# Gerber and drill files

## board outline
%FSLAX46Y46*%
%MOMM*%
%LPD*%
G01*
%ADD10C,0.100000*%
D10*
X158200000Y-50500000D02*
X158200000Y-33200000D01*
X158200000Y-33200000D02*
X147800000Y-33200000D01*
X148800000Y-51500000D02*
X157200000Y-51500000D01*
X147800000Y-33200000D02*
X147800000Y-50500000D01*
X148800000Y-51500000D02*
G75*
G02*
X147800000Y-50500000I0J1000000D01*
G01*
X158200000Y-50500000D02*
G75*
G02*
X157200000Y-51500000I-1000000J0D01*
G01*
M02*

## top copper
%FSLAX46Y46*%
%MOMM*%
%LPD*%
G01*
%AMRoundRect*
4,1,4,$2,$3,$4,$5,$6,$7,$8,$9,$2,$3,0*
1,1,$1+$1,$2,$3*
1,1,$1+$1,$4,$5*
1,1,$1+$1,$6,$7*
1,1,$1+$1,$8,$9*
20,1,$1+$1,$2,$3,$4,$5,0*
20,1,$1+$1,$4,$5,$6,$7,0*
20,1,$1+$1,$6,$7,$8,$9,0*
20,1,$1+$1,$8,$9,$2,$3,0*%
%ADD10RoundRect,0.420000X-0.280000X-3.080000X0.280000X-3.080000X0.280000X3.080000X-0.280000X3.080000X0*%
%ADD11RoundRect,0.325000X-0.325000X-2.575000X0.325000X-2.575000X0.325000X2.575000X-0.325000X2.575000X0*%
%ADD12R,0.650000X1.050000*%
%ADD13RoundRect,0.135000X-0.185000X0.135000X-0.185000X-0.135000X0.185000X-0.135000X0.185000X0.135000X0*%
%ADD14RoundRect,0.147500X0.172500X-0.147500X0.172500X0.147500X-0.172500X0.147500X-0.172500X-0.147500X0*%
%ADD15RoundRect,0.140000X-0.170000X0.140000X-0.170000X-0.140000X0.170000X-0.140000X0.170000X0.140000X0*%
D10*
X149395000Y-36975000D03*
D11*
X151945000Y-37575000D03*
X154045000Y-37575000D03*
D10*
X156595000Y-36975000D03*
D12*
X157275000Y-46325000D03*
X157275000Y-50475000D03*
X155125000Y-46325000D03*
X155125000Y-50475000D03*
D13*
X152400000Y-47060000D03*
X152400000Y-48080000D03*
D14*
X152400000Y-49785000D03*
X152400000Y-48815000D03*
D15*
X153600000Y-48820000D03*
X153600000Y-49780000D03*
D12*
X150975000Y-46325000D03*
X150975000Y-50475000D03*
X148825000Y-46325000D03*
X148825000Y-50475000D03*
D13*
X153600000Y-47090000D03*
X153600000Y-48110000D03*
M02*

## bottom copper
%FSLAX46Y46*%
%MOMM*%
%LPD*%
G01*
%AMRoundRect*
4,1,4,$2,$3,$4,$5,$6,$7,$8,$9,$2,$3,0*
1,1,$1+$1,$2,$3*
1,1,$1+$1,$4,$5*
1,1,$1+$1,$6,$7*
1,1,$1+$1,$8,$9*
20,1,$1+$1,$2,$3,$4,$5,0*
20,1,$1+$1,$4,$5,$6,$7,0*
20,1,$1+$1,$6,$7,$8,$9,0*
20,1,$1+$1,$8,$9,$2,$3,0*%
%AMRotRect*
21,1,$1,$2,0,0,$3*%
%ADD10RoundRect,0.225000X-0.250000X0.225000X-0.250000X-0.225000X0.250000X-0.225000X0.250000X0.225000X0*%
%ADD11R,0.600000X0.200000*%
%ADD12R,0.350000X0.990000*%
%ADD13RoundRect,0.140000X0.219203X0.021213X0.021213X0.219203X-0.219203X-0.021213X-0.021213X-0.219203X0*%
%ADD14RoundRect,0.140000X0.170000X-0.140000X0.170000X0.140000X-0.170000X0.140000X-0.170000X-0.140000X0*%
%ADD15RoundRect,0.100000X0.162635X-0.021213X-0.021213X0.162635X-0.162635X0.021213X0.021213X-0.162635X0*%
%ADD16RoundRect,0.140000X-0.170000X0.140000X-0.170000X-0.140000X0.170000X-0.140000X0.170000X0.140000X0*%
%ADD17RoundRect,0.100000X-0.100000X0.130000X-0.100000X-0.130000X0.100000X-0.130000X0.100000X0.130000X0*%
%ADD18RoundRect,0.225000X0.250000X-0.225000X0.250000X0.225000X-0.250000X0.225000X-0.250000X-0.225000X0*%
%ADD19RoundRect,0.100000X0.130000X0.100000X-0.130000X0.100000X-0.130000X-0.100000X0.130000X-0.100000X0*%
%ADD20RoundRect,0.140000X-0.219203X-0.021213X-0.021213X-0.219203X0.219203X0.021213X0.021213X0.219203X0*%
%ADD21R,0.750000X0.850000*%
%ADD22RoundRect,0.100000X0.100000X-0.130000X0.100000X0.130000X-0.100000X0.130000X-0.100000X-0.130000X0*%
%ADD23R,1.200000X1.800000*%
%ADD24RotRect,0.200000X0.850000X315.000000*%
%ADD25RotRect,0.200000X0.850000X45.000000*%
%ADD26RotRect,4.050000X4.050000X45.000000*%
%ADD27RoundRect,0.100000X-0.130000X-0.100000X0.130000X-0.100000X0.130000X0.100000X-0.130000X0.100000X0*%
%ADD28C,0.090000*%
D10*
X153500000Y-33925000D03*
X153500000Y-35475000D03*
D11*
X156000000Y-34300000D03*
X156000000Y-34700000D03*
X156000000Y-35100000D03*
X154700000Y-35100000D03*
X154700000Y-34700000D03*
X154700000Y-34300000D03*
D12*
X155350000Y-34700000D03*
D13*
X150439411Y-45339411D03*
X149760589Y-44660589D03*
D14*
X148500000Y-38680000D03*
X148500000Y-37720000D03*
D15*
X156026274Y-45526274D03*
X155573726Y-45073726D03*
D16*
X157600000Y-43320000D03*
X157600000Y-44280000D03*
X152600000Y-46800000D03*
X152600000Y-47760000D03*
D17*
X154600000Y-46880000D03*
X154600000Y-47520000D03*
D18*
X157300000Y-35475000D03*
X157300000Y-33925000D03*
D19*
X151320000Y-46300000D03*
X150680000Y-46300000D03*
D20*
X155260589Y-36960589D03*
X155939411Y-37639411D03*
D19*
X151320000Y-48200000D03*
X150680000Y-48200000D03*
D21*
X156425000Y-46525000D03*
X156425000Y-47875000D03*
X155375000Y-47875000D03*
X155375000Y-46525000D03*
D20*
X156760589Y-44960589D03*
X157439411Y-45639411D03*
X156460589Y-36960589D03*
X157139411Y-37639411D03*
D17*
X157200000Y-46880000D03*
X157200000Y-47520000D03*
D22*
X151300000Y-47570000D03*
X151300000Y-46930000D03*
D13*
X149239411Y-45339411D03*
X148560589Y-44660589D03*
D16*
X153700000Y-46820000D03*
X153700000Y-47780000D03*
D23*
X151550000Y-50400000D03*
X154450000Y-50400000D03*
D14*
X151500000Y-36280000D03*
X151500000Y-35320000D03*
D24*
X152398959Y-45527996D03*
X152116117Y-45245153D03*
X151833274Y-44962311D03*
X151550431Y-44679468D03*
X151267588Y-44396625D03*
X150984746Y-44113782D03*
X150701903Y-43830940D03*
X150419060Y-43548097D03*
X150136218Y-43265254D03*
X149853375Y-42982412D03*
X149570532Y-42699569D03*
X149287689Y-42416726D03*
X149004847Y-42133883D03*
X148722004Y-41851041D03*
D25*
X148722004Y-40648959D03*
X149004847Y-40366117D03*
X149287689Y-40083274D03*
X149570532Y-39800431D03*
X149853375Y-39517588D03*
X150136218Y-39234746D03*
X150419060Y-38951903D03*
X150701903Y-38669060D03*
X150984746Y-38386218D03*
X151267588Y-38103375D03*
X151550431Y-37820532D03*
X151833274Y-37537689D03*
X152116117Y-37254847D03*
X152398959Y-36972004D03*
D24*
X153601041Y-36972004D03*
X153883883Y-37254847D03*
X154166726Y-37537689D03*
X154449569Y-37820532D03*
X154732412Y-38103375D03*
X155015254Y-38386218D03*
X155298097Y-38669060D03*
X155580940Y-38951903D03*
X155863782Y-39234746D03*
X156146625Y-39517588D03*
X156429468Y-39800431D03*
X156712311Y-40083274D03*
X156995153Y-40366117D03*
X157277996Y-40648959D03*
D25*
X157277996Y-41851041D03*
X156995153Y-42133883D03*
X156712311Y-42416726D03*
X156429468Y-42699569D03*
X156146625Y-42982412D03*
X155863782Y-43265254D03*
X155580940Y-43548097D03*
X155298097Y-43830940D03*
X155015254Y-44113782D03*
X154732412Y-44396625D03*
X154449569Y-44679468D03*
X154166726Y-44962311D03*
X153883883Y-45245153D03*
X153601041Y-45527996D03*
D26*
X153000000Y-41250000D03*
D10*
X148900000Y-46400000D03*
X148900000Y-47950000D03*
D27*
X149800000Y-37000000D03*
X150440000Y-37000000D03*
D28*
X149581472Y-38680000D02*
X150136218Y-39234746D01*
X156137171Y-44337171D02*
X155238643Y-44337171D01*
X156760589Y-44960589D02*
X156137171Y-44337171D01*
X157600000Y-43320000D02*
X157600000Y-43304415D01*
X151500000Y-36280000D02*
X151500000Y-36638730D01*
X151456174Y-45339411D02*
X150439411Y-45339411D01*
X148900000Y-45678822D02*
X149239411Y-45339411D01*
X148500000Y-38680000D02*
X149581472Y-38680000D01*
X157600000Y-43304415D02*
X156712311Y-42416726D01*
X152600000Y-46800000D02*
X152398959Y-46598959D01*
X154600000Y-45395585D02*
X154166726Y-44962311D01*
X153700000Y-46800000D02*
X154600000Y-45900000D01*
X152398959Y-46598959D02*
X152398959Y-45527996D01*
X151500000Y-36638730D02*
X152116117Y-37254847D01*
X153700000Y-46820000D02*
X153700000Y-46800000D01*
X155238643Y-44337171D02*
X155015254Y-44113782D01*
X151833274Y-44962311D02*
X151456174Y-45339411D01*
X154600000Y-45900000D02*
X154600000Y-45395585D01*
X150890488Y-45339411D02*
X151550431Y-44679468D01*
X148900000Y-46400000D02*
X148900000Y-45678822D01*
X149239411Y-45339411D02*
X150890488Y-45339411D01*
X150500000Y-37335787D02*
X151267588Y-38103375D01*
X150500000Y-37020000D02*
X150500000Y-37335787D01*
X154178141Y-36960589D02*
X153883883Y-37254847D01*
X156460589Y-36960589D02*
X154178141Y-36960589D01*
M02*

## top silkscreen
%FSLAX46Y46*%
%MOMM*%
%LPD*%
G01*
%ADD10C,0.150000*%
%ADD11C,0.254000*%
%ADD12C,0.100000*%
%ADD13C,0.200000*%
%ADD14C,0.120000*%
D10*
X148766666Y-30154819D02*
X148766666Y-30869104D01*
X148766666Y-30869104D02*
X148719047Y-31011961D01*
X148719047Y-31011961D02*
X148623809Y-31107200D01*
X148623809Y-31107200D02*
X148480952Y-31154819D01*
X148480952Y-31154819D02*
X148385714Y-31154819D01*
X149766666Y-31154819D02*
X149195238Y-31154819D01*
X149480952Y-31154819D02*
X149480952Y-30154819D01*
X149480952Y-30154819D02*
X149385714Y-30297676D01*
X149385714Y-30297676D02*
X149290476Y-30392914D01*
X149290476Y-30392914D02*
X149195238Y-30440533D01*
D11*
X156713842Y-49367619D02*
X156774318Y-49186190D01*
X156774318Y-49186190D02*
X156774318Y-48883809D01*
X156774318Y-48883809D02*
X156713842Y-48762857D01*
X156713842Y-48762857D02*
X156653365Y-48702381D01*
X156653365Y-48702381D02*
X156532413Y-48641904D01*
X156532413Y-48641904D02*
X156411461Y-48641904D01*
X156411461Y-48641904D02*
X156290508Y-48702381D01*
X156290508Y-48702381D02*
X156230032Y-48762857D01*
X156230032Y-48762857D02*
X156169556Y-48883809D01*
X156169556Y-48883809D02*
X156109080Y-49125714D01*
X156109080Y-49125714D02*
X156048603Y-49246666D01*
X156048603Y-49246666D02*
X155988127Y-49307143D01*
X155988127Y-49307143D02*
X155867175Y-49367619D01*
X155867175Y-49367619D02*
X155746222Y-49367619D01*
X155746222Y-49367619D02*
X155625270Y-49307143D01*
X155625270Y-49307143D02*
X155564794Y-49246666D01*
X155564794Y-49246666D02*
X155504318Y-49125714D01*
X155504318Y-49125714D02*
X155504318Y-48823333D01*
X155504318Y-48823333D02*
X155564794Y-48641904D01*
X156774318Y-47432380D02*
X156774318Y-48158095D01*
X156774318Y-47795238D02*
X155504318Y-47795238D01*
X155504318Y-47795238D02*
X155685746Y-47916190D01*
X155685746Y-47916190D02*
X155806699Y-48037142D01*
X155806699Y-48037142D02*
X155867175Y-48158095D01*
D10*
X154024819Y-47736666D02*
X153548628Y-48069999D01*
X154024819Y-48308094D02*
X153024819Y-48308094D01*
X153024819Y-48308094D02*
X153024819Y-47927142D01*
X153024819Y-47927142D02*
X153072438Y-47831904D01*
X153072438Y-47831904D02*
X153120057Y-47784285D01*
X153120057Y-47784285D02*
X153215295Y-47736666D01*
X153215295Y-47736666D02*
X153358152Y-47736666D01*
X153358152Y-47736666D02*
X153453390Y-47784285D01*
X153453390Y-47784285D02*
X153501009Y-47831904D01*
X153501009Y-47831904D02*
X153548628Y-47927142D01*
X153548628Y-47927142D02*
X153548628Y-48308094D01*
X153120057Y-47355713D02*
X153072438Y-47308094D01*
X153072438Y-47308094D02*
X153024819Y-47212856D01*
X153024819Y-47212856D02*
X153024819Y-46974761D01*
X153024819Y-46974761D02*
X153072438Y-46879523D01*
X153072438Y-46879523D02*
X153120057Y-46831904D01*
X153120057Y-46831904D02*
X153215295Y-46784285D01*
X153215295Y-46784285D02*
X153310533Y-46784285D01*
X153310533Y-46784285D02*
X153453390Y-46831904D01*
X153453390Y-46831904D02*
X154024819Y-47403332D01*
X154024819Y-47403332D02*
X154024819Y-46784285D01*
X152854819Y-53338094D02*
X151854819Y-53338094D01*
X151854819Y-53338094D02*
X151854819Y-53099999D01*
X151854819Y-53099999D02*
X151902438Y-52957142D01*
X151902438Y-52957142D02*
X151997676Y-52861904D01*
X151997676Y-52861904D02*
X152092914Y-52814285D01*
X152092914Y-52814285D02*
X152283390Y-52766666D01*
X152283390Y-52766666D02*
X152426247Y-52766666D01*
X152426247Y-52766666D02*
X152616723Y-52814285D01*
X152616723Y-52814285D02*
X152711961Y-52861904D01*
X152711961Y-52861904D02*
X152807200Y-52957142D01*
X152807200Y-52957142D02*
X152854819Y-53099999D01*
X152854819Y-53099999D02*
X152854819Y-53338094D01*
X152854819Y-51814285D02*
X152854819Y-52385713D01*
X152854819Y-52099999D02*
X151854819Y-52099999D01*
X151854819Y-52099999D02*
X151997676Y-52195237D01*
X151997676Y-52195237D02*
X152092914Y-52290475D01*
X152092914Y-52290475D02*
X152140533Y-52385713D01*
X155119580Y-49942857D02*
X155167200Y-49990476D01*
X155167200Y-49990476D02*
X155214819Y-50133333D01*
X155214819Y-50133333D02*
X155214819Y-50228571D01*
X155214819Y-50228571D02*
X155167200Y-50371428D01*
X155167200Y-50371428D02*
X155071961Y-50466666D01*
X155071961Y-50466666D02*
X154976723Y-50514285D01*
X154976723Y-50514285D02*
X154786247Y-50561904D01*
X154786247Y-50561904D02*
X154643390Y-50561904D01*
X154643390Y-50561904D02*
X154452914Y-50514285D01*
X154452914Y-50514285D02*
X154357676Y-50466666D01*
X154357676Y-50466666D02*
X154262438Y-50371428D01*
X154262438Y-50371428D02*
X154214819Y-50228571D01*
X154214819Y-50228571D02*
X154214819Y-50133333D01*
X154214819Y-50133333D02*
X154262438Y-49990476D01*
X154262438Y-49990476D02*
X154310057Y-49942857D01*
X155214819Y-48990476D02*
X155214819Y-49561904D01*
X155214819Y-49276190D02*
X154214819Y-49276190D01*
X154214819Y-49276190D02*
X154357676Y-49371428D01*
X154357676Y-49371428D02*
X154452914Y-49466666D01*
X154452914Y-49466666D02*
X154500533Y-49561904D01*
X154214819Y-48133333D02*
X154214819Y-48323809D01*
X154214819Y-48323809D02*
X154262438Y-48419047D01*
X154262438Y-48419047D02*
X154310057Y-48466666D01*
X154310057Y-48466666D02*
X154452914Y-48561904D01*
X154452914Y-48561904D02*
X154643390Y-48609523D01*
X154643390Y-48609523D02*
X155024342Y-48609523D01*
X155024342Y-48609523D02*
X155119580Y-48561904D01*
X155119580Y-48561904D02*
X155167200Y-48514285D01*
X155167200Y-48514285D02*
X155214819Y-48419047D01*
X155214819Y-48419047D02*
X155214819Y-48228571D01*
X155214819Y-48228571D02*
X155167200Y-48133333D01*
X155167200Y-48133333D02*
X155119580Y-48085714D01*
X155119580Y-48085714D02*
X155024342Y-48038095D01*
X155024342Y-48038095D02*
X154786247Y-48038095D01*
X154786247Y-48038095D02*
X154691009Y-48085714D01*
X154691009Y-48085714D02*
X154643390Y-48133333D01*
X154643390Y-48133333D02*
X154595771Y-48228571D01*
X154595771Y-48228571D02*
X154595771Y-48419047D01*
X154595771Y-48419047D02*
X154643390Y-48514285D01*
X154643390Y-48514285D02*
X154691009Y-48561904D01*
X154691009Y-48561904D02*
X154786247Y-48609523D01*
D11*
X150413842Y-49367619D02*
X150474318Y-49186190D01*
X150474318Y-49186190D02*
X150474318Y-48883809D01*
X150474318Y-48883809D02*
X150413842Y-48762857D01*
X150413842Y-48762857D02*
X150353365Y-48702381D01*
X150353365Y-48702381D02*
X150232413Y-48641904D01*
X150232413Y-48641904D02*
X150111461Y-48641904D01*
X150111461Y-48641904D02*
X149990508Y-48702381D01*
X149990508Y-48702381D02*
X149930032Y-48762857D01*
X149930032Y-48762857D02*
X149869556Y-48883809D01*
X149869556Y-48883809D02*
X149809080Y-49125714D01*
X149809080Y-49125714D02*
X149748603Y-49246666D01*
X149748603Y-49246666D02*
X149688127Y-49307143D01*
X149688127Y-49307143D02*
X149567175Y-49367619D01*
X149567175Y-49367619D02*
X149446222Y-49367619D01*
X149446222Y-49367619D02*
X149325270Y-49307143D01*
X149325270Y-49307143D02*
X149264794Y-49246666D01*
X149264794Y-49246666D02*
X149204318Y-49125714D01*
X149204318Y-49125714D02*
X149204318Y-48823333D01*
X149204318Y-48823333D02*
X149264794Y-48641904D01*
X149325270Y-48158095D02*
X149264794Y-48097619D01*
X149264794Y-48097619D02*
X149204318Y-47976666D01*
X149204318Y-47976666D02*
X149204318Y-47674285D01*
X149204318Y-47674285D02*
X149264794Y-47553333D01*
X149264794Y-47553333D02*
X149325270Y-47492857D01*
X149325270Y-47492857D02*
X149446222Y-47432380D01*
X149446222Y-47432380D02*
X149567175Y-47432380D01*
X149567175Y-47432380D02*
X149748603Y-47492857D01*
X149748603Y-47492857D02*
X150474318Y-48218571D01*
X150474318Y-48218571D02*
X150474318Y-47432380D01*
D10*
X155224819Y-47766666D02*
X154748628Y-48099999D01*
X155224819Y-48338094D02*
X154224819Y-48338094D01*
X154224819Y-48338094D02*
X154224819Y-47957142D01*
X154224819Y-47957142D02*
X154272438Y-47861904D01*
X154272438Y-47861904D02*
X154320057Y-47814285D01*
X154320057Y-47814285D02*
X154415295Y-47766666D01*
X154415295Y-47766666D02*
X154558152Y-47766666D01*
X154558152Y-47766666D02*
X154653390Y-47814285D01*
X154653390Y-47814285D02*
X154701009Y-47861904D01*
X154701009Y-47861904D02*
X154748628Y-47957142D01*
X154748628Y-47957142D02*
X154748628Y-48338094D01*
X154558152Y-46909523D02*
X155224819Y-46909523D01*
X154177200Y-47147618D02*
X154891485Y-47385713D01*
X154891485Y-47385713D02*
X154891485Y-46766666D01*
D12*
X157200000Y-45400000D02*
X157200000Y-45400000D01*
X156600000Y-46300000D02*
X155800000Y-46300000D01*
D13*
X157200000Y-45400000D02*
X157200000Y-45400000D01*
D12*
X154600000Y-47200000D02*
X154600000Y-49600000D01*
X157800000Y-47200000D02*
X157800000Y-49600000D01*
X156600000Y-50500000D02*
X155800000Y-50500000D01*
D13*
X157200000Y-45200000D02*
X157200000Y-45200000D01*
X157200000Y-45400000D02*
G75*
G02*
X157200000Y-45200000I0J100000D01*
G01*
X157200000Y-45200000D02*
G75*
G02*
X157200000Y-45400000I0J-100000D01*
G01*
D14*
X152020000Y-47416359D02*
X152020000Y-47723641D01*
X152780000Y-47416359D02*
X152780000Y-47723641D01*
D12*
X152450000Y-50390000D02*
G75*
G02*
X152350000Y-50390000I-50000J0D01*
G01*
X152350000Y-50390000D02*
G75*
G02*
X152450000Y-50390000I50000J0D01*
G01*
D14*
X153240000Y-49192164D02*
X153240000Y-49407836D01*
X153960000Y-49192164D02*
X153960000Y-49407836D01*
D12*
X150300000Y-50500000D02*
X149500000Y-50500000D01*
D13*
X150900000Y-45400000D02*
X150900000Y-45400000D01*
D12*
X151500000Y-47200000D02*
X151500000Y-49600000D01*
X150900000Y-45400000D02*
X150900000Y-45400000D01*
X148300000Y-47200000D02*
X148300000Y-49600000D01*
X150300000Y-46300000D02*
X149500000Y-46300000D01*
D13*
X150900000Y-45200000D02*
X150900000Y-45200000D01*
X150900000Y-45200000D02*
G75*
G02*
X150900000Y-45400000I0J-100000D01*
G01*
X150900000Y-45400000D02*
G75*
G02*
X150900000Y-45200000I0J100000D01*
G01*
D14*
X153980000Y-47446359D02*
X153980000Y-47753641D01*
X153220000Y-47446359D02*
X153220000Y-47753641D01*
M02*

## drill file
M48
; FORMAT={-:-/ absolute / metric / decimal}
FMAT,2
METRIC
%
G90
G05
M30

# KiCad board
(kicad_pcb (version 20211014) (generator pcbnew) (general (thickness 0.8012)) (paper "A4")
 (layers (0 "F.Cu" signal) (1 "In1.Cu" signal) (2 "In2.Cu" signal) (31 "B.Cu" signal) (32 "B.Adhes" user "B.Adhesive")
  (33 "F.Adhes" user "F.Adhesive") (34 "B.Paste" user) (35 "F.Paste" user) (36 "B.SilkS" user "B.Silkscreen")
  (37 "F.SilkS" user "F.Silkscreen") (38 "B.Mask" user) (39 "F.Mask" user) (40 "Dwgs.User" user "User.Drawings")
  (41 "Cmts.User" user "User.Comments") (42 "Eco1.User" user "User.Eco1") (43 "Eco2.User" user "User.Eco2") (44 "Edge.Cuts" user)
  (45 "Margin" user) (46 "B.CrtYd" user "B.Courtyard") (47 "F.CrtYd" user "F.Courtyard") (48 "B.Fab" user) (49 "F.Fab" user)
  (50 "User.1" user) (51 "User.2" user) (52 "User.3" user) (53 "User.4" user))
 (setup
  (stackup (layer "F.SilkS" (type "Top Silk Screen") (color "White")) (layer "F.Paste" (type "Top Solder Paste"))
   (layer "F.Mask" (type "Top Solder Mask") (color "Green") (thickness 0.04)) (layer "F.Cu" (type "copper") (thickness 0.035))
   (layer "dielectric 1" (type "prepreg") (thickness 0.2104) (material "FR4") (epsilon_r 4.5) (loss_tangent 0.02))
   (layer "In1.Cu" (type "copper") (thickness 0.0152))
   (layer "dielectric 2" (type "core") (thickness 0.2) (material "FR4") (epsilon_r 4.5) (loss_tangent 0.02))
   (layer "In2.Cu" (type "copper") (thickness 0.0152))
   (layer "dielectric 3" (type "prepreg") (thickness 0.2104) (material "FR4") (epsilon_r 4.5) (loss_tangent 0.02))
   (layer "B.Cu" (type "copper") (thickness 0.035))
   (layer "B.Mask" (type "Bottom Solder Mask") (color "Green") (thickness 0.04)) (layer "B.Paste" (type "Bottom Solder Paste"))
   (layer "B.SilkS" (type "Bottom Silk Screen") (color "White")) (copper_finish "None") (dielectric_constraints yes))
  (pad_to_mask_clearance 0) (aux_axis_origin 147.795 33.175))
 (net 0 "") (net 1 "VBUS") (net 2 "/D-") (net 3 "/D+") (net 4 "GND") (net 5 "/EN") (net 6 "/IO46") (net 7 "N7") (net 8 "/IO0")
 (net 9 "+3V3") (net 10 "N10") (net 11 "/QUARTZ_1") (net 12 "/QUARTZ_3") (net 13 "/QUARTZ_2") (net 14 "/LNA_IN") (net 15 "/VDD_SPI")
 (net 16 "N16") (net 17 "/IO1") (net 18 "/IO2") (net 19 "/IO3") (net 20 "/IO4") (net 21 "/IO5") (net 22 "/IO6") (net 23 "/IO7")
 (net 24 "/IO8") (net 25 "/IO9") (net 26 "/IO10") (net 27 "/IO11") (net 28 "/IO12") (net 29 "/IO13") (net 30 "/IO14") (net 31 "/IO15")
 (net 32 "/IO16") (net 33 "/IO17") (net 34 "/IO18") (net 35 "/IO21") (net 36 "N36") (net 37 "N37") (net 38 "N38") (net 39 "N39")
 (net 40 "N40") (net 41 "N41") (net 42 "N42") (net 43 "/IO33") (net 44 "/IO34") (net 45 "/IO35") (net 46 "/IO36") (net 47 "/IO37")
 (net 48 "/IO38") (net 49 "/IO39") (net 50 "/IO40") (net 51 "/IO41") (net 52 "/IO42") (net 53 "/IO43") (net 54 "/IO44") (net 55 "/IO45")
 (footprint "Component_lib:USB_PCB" (layer "F.Cu") (at 152.995 44.375)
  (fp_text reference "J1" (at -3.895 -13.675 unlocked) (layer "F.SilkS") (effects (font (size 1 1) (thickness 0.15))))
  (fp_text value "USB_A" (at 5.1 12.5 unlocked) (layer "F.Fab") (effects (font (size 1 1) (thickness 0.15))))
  (pad "1" smd roundrect (at -3.6 -7.4) (size 1.4 7) (layers "F.Cu" "F.Paste" "F.Mask") (roundrect_rratio 0.3) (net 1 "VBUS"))
  (pad "2" smd roundrect (at -1.05 -6.8) (size 1.3 5.8) (layers "F.Cu" "F.Paste" "F.Mask") (roundrect_rratio 0.25) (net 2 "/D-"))
  (pad "3" smd roundrect (at 1.05 -6.8) (size 1.3 5.8) (layers "F.Cu" "F.Paste" "F.Mask") (roundrect_rratio 0.25) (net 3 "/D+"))
  (pad "4" smd roundrect (at 3.6 -7.4) (size 1.4 7) (layers "F.Cu" "F.Paste" "F.Mask") (roundrect_rratio 0.3) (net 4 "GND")))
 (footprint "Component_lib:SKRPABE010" (layer "F.Cu") (at 156.2 48.4 -90)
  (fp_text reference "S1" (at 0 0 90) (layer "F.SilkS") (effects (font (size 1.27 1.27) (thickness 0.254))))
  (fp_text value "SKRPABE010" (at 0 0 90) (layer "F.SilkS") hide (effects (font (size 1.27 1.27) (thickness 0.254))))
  (fp_line (start -3 -1) (end -3 -1) (layer "F.SilkS") (width 0.1))
  (fp_line (start -2.1 -0.4) (end -2.1 0.4) (layer "F.SilkS") (width 0.1))
  (fp_line (start -3 -1) (end -3 -1) (layer "F.SilkS") (width 0.2))
  (fp_line (start -1.2 1.6) (end 1.2 1.6) (layer "F.SilkS") (width 0.1))
  (fp_line (start -1.2 -1.6) (end 1.2 -1.6) (layer "F.SilkS") (width 0.1))
  (fp_line (start 2.1 -0.4) (end 2.1 0.4) (layer "F.SilkS") (width 0.1))
  (fp_line (start -3.2 -1) (end -3.2 -1) (layer "F.SilkS") (width 0.2))
  (fp_arc (start -3 -1) (mid -3.1 -0.9) (end -3.2 -1) (layer "F.SilkS") (width 0.2))
  (fp_arc (start -3.2 -1) (mid -3.1 -1.1) (end -3 -1) (layer "F.SilkS") (width 0.2))
  (pad "1" smd rect (at -2.075 -1.075) (size 0.65 1.05) (layers "F.Cu" "F.Paste" "F.Mask") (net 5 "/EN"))
  (pad "2" smd rect (at 2.075 -1.075) (size 0.65 1.05) (layers "F.Cu" "F.Paste" "F.Mask") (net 4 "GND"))
  (pad "3" smd rect (at -2.075 1.075) (size 0.65 1.05) (layers "F.Cu" "F.Paste" "F.Mask"))
  (pad "4" smd rect (at 2.075 1.075) (size 0.65 1.05) (layers "F.Cu" "F.Paste" "F.Mask")))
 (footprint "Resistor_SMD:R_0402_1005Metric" (layer "F.Cu") (at 152.4 47.57 -90)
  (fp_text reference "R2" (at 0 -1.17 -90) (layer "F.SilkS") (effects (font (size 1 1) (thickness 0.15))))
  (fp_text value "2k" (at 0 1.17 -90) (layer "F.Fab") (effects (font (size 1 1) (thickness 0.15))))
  (fp_line (start -0.153641 0.38) (end 0.153641 0.38) (layer "F.SilkS") (width 0.12))
  (fp_line (start -0.153641 -0.38) (end 0.153641 -0.38) (layer "F.SilkS") (width 0.12))
  (pad "1" smd roundrect (at -0.51 0 270) (size 0.54 0.64) (layers "F.Cu" "F.Paste" "F.Mask") (roundrect_rratio 0.25) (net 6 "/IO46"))
  (pad "2" smd roundrect (at 0.51 0 270) (size 0.54 0.64) (layers "F.Cu" "F.Paste" "F.Mask") (roundrect_rratio 0.25) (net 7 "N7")))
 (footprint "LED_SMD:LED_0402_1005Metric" (layer "F.Cu") (at 152.4 49.3 90)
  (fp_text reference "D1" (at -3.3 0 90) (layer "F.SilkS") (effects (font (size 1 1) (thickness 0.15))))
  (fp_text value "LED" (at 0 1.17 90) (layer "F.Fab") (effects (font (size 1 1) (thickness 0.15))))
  (fp_circle (center -1.09 0) (end -1.04 0) (layer "F.SilkS") (width 0.1) (fill none))
  (pad "1" smd roundrect (at -0.485 0 90) (size 0.59 0.64) (layers "F.Cu" "F.Paste" "F.Mask") (roundrect_rratio 0.25) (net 4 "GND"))
  (pad "2" smd roundrect (at 0.485 0 90) (size 0.59 0.64) (layers "F.Cu" "F.Paste" "F.Mask") (roundrect_rratio 0.25) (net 7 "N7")))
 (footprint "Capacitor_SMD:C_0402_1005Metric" (layer "F.Cu") (at 153.6 49.3 -90)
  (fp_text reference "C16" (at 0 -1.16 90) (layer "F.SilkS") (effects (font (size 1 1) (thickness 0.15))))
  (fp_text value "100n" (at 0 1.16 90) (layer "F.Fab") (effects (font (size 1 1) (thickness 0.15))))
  (fp_line (start -0.107836 0.36) (end 0.107836 0.36) (layer "F.SilkS") (width 0.12))
  (fp_line (start -0.107836 -0.36) (end 0.107836 -0.36) (layer "F.SilkS") (width 0.12))
  (pad "1" smd roundrect (at -0.48 0 270) (size 0.56 0.62) (layers "F.Cu" "F.Paste" "F.Mask") (roundrect_rratio 0.25) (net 5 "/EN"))
  (pad "2" smd roundrect (at 0.48 0 270) (size 0.56 0.62) (layers "F.Cu" "F.Paste" "F.Mask") (roundrect_rratio 0.25) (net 4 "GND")))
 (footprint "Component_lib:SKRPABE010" (layer "F.Cu") (at 149.9 48.4 -90)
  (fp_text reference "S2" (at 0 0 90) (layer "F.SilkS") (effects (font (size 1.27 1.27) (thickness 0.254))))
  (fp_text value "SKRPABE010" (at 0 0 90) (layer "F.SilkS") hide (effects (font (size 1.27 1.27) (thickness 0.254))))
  (fp_line (start 2.1 -0.4) (end 2.1 0.4) (layer "F.SilkS") (width 0.1))
  (fp_line (start -3 -1) (end -3 -1) (layer "F.SilkS") (width 0.2))
  (fp_line (start -1.2 -1.6) (end 1.2 -1.6) (layer "F.SilkS") (width 0.1))
  (fp_line (start -3 -1) (end -3 -1) (layer "F.SilkS") (width 0.1))
  (fp_line (start -1.2 1.6) (end 1.2 1.6) (layer "F.SilkS") (width 0.1))
  (fp_line (start -2.1 -0.4) (end -2.1 0.4) (layer "F.SilkS") (width 0.1))
  (fp_line (start -3.2 -1) (end -3.2 -1) (layer "F.SilkS") (width 0.2))
  (fp_arc (start -3.2 -1) (mid -3.1 -1.1) (end -3 -1) (layer "F.SilkS") (width 0.2))
  (fp_arc (start -3 -1) (mid -3.1 -0.9) (end -3.2 -1) (layer "F.SilkS") (width 0.2))
  (pad "1" smd rect (at -2.075 -1.075) (size 0.65 1.05) (layers "F.Cu" "F.Paste" "F.Mask") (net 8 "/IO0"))
  (pad "2" smd rect (at 2.075 -1.075) (size 0.65 1.05) (layers "F.Cu" "F.Paste" "F.Mask") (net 4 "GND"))
  (pad "3" smd rect (at -2.075 1.075) (size 0.65 1.05) (layers "F.Cu" "F.Paste" "F.Mask"))
  (pad "4" smd rect (at 2.075 1.075) (size 0.65 1.05) (layers "F.Cu" "F.Paste" "F.Mask")))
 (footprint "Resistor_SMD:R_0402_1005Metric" (layer "F.Cu") (at 153.6 47.6 -90)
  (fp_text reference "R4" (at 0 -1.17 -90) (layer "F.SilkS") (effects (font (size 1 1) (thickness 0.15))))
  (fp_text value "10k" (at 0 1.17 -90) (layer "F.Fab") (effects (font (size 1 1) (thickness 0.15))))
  (fp_line (start -0.153641 -0.38) (end 0.153641 -0.38) (layer "F.SilkS") (width 0.12))
  (fp_line (start -0.153641 0.38) (end 0.153641 0.38) (layer "F.SilkS") (width 0.12))
  (pad "1" smd roundrect (at -0.51 0 270) (size 0.54 0.64) (layers "F.Cu" "F.Paste" "F.Mask") (roundrect_rratio 0.25) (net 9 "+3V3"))
  (pad "2" smd roundrect (at 0.51 0 270) (size 0.54 0.64) (layers "F.Cu" "F.Paste" "F.Mask") (roundrect_rratio 0.25) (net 5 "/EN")))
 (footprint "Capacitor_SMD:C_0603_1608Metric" (layer "B.Cu") (at 153.5 34.7 -90)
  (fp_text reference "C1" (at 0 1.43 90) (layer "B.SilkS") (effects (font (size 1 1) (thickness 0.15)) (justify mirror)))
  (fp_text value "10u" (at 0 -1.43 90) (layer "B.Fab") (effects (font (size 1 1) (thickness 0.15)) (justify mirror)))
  (pad "1" smd roundrect (at -0.775 0 270) (size 0.9 0.95) (layers "B.Cu" "B.Paste" "B.Mask") (roundrect_rratio 0.25) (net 1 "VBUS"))
  (pad "2" smd roundrect (at 0.775 0 270) (size 0.9 0.95) (layers "B.Cu" "B.Paste" "B.Mask") (roundrect_rratio 0.25) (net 4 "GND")))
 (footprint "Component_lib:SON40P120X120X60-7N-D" (layer "B.Cu") (at 155.35 34.7 180)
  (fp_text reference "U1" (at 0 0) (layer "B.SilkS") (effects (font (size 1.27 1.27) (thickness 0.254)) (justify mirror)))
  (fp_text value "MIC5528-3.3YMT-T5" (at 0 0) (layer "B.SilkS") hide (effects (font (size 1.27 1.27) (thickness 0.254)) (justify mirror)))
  (pad "1" smd rect locked (at -0.65 0.4 90) (size 0.2 0.6) (layers "B.Cu" "B.Paste" "B.Mask") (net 9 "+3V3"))
  (pad "2" smd rect locked (at -0.65 0 90) (size 0.2 0.6) (layers "B.Cu" "B.Paste" "B.Mask") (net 9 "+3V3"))
  (pad "3" smd rect locked (at -0.65 -0.4 90) (size 0.2 0.6) (layers "B.Cu" "B.Paste" "B.Mask") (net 4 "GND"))
  (pad "4" smd rect locked (at 0.65 -0.4 90) (size 0.2 0.6) (layers "B.Cu" "B.Paste" "B.Mask") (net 1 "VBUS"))
  (pad "5" smd rect locked (at 0.65 0 90) (size 0.2 0.6) (layers "B.Cu" "B.Paste" "B.Mask") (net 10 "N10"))
  (pad "6" smd rect locked (at 0.65 0.4 90) (size 0.2 0.6) (layers "B.Cu" "B.Paste" "B.Mask") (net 1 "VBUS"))
  (pad "7" smd rect locked (at 0 0 180) (size 0.35 0.99) (layers "B.Cu" "B.Paste" "B.Mask") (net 4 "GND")))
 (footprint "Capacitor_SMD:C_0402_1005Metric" (layer "B.Cu") (at 150.1 45 135)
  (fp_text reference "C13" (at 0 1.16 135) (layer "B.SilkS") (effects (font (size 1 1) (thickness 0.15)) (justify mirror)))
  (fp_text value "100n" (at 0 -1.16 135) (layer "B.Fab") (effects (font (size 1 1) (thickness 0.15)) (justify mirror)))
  (pad "1" smd roundrect (at -0.48 0 135) (size 0.56 0.62) (layers "B.Cu" "B.Paste" "B.Mask") (roundrect_rratio 0.25) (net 9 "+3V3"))
  (pad "2" smd roundrect (at 0.48 0 135) (size 0.56 0.62) (layers "B.Cu" "B.Paste" "B.Mask") (roundrect_rratio 0.25) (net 4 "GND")))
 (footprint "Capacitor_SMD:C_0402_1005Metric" (layer "B.Cu") (at 148.5 38.2 90)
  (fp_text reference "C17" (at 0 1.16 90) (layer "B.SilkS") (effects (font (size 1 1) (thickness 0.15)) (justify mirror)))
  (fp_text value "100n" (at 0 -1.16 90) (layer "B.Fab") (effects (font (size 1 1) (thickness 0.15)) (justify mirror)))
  (pad "1" smd roundrect (at -0.48 0 90) (size 0.56 0.62) (layers "B.Cu" "B.Paste" "B.Mask") (roundrect_rratio 0.25) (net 9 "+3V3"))
  (pad "2" smd roundrect (at 0.48 0 90) (size 0.56 0.62) (layers "B.Cu" "B.Paste" "B.Mask") (roundrect_rratio 0.25) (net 4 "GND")))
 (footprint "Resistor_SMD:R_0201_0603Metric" (layer "B.Cu") (at 155.8 45.3 135)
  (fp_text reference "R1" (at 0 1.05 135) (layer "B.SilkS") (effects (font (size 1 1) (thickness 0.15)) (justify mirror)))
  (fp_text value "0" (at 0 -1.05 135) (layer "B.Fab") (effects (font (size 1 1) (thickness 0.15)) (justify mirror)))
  (pad "" smd roundrect (at -0.345 0 135) (size 0.318 0.36) (layers "B.Paste") (roundrect_rratio 0.25))
  (pad "" smd roundrect (at 0.345 0 135) (size 0.318 0.36) (layers "B.Paste") (roundrect_rratio 0.25))
  (pad "1" smd roundrect (at -0.32 0 135) (size 0.46 0.4) (layers "B.Cu" "B.Mask") (roundrect_rratio 0.25) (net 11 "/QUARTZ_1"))
  (pad "2" smd roundrect (at 0.32 0 135) (size 0.46 0.4) (layers "B.Cu" "B.Mask") (roundrect_rratio 0.25) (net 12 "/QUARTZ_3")))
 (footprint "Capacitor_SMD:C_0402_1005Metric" (layer "B.Cu") (at 157.6 43.8 -90)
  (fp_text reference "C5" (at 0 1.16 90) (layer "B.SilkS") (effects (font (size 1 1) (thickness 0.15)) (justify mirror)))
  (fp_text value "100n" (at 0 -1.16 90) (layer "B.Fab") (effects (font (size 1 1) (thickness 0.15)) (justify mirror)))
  (pad "1" smd roundrect (at -0.48 0 270) (size 0.56 0.62) (layers "B.Cu" "B.Paste" "B.Mask") (roundrect_rratio 0.25) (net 9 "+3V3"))
  (pad "2" smd roundrect (at 0.48 0 270) (size 0.56 0.62) (layers "B.Cu" "B.Paste" "B.Mask") (roundrect_rratio 0.25) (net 4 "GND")))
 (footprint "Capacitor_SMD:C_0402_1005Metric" (layer "B.Cu") (at 152.6 47.28 -90)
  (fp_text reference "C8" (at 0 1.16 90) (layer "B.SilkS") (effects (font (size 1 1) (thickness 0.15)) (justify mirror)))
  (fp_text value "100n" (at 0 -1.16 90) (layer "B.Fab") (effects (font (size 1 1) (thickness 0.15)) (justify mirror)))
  (pad "1" smd roundrect (at -0.48 0 270) (size 0.56 0.62) (layers "B.Cu" "B.Paste" "B.Mask") (roundrect_rratio 0.25) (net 9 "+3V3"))
  (pad "2" smd roundrect (at 0.48 0 270) (size 0.56 0.62) (layers "B.Cu" "B.Paste" "B.Mask") (roundrect_rratio 0.25) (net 4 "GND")))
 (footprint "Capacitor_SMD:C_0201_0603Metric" (layer "B.Cu") (at 154.6 47.2 -90)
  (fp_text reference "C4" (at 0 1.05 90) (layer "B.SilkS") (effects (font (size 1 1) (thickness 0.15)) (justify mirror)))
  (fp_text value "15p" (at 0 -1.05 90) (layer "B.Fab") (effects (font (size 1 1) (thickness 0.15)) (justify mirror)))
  (pad "" smd roundrect (at 0.345 0 270) (size 0.318 0.36) (layers "B.Paste") (roundrect_rratio 0.25))
  (pad "" smd roundrect (at -0.345 0 270) (size 0.318 0.36) (layers "B.Paste") (roundrect_rratio 0.25))
  (pad "1" smd roundrect (at -0.32 0 270) (size 0.46 0.4) (layers "B.Cu" "B.Mask") (roundrect_rratio 0.25) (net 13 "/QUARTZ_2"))
  (pad "2" smd roundrect (at 0.32 0 270) (size 0.46 0.4) (layers "B.Cu" "B.Mask") (roundrect_rratio 0.25) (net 4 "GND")))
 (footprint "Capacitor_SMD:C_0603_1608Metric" (layer "B.Cu") (at 157.3 34.7 90)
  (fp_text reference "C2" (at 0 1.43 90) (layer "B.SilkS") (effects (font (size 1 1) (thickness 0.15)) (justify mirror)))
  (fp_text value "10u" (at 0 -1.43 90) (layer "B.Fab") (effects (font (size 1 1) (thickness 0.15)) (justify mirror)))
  (pad "1" smd roundrect (at -0.775 0 90) (size 0.9 0.95) (layers "B.Cu" "B.Paste" "B.Mask") (roundrect_rratio 0.25) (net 9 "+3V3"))
  (pad "2" smd roundrect (at 0.775 0 90) (size 0.9 0.95) (layers "B.Cu" "B.Paste" "B.Mask") (roundrect_rratio 0.25) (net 4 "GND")))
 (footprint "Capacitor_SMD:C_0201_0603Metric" (layer "B.Cu") (at 151 46.3 180)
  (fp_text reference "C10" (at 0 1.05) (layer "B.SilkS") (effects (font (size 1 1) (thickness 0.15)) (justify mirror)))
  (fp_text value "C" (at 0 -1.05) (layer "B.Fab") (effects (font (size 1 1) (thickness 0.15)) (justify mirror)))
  (pad "" smd roundrect (at -0.345 0 180) (size 0.318 0.36) (layers "B.Paste") (roundrect_rratio 0.25))
  (pad "" smd roundrect (at 0.345 0 180) (size 0.318 0.36) (layers "B.Paste") (roundrect_rratio 0.25))
  (pad "1" smd roundrect (at -0.32 0 180) (size 0.46 0.4) (layers "B.Cu" "B.Mask") (roundrect_rratio 0.25) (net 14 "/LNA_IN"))
  (pad "2" smd roundrect (at 0.32 0 180) (size 0.46 0.4) (layers "B.Cu" "B.Mask") (roundrect_rratio 0.25) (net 4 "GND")))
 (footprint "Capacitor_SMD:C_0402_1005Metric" (layer "B.Cu") (at 155.6 37.3 -45)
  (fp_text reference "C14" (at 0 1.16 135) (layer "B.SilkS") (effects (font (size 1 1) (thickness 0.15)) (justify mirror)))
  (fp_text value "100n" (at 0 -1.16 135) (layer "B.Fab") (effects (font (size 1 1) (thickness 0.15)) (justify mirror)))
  (pad "1" smd roundrect (at -0.48 0 315) (size 0.56 0.62) (layers "B.Cu" "B.Paste" "B.Mask") (roundrect_rratio 0.25) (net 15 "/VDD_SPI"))
  (pad "2" smd roundrect (at 0.48 0 315) (size 0.56 0.62) (layers "B.Cu" "B.Paste" "B.Mask") (roundrect_rratio 0.25) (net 4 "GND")))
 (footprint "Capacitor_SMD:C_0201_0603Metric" (layer "B.Cu") (at 151 48.2 180)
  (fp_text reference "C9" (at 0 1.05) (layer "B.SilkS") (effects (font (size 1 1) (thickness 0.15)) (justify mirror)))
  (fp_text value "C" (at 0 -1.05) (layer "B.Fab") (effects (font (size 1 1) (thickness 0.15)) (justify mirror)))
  (pad "" smd roundrect (at 0.345 0 180) (size 0.318 0.36) (layers "B.Paste") (roundrect_rratio 0.25))
  (pad "" smd roundrect (at -0.345 0 180) (size 0.318 0.36) (layers "B.Paste") (roundrect_rratio 0.25))
  (pad "1" smd roundrect (at -0.32 0 180) (size 0.46 0.4) (layers "B.Cu" "B.Mask") (roundrect_rratio 0.25) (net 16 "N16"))
  (pad "2" smd roundrect (at 0.32 0 180) (size 0.46 0.4) (layers "B.Cu" "B.Mask") (roundrect_rratio 0.25) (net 4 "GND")))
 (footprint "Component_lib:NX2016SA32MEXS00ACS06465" (layer "B.Cu") (at 155.9 47.2 -90)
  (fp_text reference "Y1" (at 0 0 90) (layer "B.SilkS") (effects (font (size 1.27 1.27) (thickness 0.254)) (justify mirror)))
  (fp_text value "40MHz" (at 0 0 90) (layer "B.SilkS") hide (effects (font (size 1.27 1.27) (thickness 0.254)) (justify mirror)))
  (pad "1" smd rect (at -0.675 -0.525 180) (size 0.75 0.85) (layers "B.Cu" "B.Paste" "B.Mask") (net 11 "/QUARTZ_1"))
  (pad "2" smd rect (at 0.675 -0.525 180) (size 0.75 0.85) (layers "B.Cu" "B.Paste" "B.Mask") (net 4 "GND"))
  (pad "3" smd rect (at 0.675 0.525 180) (size 0.75 0.85) (layers "B.Cu" "B.Paste" "B.Mask") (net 4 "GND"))
  (pad "4" smd rect (at -0.675 0.525 180) (size 0.75 0.85) (layers "B.Cu" "B.Paste" "B.Mask") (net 13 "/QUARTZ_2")))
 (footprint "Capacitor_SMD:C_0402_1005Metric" (layer "B.Cu") (at 157.1 45.3 -45)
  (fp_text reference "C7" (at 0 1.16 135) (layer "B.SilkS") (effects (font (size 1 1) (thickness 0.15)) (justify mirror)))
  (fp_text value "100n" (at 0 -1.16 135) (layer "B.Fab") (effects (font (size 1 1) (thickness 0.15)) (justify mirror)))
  (pad "1" smd roundrect (at -0.48 0 315) (size 0.56 0.62) (layers "B.Cu" "B.Paste" "B.Mask") (roundrect_rratio 0.25) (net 9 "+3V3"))
  (pad "2" smd roundrect (at 0.48 0 315) (size 0.56 0.62) (layers "B.Cu" "B.Paste" "B.Mask") (roundrect_rratio 0.25) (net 4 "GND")))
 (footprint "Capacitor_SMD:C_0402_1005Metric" (layer "B.Cu") (at 156.8 37.3 -45)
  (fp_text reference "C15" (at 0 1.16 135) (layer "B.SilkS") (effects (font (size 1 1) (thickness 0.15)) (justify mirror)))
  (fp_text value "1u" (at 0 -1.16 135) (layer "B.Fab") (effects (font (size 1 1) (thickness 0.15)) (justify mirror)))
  (pad "1" smd roundrect (at -0.48 0 315) (size 0.56 0.62) (layers "B.Cu" "B.Paste" "B.Mask") (roundrect_rratio 0.25) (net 15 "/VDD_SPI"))
  (pad "2" smd roundrect (at 0.48 0 315) (size 0.56 0.62) (layers "B.Cu" "B.Paste" "B.Mask") (roundrect_rratio 0.25) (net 4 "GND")))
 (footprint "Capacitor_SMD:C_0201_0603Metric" (layer "B.Cu") (at 157.2 47.2 -90)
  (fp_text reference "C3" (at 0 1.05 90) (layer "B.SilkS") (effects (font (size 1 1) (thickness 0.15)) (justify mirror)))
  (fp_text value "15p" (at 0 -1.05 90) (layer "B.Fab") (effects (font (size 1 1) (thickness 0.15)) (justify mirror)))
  (pad "" smd roundrect (at -0.345 0 270) (size 0.318 0.36) (layers "B.Paste") (roundrect_rratio 0.25))
  (pad "" smd roundrect (at 0.345 0 270) (size 0.318 0.36) (layers "B.Paste") (roundrect_rratio 0.25))
  (pad "1" smd roundrect (at -0.32 0 270) (size 0.46 0.4) (layers "B.Cu" "B.Mask") (roundrect_rratio 0.25) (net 11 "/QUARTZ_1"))
  (pad "2" smd roundrect (at 0.32 0 270) (size 0.46 0.4) (layers "B.Cu" "B.Mask") (roundrect_rratio 0.25) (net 4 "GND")))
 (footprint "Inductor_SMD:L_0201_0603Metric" (layer "B.Cu") (at 151.3 47.25 90)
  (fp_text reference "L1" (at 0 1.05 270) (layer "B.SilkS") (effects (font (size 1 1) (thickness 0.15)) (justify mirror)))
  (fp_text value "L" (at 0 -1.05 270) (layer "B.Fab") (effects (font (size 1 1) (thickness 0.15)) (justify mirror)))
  (pad "" smd roundrect (at 0.345 0 90) (size 0.318 0.36) (layers "B.Paste") (roundrect_rratio 0.25))
  (pad "" smd roundrect (at -0.345 0 90) (size 0.318 0.36) (layers "B.Paste") (roundrect_rratio 0.25))
  (pad "1" smd roundrect (at -0.32 0 90) (size 0.46 0.4) (layers "B.Cu" "B.Mask") (roundrect_rratio 0.25) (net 16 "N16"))
  (pad "2" smd roundrect (at 0.32 0 90) (size 0.46 0.4) (layers "B.Cu" "B.Mask") (roundrect_rratio 0.25) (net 14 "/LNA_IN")))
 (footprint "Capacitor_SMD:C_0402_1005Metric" (layer "B.Cu") (at 148.9 45 135)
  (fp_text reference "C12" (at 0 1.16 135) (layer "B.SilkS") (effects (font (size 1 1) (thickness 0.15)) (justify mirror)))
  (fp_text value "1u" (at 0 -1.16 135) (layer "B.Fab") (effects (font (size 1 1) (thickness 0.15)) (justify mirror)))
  (pad "1" smd roundrect (at -0.48 0 135) (size 0.56 0.62) (layers "B.Cu" "B.Paste" "B.Mask") (roundrect_rratio 0.25) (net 9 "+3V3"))
  (pad "2" smd roundrect (at 0.48 0 135) (size 0.56 0.62) (layers "B.Cu" "B.Paste" "B.Mask") (roundrect_rratio 0.25) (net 4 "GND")))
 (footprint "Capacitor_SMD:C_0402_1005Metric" (layer "B.Cu") (at 153.7 47.3 -90)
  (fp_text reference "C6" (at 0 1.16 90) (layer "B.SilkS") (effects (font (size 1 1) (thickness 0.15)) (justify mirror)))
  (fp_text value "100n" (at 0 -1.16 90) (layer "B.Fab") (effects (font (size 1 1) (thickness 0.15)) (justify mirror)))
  (pad "1" smd roundrect (at -0.48 0 270) (size 0.56 0.62) (layers "B.Cu" "B.Paste" "B.Mask") (roundrect_rratio 0.25) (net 9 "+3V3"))
  (pad "2" smd roundrect (at 0.48 0 270) (size 0.56 0.62) (layers "B.Cu" "B.Paste" "B.Mask") (roundrect_rratio 0.25) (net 4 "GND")))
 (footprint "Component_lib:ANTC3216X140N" (layer "B.Cu") (at 153 50.4)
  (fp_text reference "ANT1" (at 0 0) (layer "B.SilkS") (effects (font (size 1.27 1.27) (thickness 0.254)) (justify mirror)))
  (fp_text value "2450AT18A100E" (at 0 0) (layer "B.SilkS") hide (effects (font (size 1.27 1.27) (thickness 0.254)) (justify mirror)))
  (pad "1" smd rect (at -1.45 0) (size 1.2 1.8) (layers "B.Cu" "B.Paste" "B.Mask") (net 16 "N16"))
  (pad "2" smd rect (at 1.45 0) (size 1.2 1.8) (layers "B.Cu" "B.Paste" "B.Mask")))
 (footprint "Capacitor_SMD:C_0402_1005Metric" (layer "B.Cu") (at 151.5 35.8 90)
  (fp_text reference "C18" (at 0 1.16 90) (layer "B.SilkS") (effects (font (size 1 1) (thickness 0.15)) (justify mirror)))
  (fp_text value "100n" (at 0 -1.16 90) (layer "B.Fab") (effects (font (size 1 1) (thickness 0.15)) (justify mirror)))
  (pad "1" smd roundrect (at -0.48 0 90) (size 0.56 0.62) (layers "B.Cu" "B.Paste" "B.Mask") (roundrect_rratio 0.25) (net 9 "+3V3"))
  (pad "2" smd roundrect (at 0.48 0 90) (size 0.56 0.62) (layers "B.Cu" "B.Paste" "B.Mask") (roundrect_rratio 0.25) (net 4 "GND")))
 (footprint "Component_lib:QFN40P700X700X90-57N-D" (layer "B.Cu") (at 153 41.25 45)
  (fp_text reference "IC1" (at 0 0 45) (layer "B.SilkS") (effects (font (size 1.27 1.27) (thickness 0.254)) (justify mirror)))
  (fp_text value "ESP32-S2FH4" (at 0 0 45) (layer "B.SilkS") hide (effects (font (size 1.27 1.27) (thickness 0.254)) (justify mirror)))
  (pad "1" smd rect (at -3.45 2.6 315) (size 0.2 0.85) (layers "B.Cu" "B.Paste" "B.Mask") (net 9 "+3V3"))
  (pad "2" smd rect (at -3.45 2.2 315) (size 0.2 0.85) (layers "B.Cu" "B.Paste" "B.Mask") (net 14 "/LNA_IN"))
  (pad "3" smd rect (at -3.45 1.8 315) (size 0.2 0.85) (layers "B.Cu" "B.Paste" "B.Mask") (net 9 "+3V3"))
  (pad "4" smd rect (at -3.45 1.4 315) (size 0.2 0.85) (layers "B.Cu" "B.Paste" "B.Mask") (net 9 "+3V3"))
  (pad "5" smd rect (at -3.45 1 315) (size 0.2 0.85) (layers "B.Cu" "B.Paste" "B.Mask") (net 8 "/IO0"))
  (pad "6" smd rect (at -3.45 0.6 315) (size 0.2 0.85) (layers "B.Cu" "B.Paste" "B.Mask") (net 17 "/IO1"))
  (pad "7" smd rect (at -3.45 0.2 315) (size 0.2 0.85) (layers "B.Cu" "B.Paste" "B.Mask") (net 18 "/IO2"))
  (pad "8" smd rect (at -3.45 -0.2 315) (size 0.2 0.85) (layers "B.Cu" "B.Paste" "B.Mask") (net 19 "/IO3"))
  (pad "9" smd rect (at -3.45 -0.6 315) (size 0.2 0.85) (layers "B.Cu" "B.Paste" "B.Mask") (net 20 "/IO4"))
  (pad "10" smd rect (at -3.45 -1 315) (size 0.2 0.85) (layers "B.Cu" "B.Paste" "B.Mask") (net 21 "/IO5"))
  (pad "11" smd rect (at -3.45 -1.4 315) (size 0.2 0.85) (layers "B.Cu" "B.Paste" "B.Mask") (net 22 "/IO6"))
  (pad "12" smd rect (at -3.45 -1.8 315) (size 0.2 0.85) (layers "B.Cu" "B.Paste" "B.Mask") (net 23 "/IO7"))
  (pad "13" smd rect (at -3.45 -2.2 315) (size 0.2 0.85) (layers "B.Cu" "B.Paste" "B.Mask") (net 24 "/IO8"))
  (pad "14" smd rect (at -3.45 -2.6 315) (size 0.2 0.85) (layers "B.Cu" "B.Paste" "B.Mask") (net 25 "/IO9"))
  (pad "15" smd rect (at -2.6 -3.45 45) (size 0.2 0.85) (layers "B.Cu" "B.Paste" "B.Mask") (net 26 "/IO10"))
  (pad "16" smd rect (at -2.2 -3.45 45) (size 0.2 0.85) (layers "B.Cu" "B.Paste" "B.Mask") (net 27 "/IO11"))
  (pad "17" smd rect (at -1.8 -3.45 45) (size 0.2 0.85) (layers "B.Cu" "B.Paste" "B.Mask") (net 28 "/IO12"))
  (pad "18" smd rect (at -1.4 -3.45 45) (size 0.2 0.85) (layers "B.Cu" "B.Paste" "B.Mask") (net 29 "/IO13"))
  (pad "19" smd rect (at -1 -3.45 45) (size 0.2 0.85) (layers "B.Cu" "B.Paste" "B.Mask") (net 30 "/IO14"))
  (pad "20" smd rect (at -0.6 -3.45 45) (size 0.2 0.85) (layers "B.Cu" "B.Paste" "B.Mask") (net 9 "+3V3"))
  (pad "21" smd rect (at -0.2 -3.45 45) (size 0.2 0.85) (layers "B.Cu" "B.Paste" "B.Mask") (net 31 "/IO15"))
  (pad "22" smd rect (at 0.2 -3.45 45) (size 0.2 0.85) (layers "B.Cu" "B.Paste" "B.Mask") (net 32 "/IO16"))
  (pad "23" smd rect (at 0.6 -3.45 45) (size 0.2 0.85) (layers "B.Cu" "B.Paste" "B.Mask") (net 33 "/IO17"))
  (pad "24" smd rect (at 1 -3.45 45) (size 0.2 0.85) (layers "B.Cu" "B.Paste" "B.Mask") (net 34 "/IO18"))
  (pad "25" smd rect (at 1.4 -3.45 45) (size 0.2 0.85) (layers "B.Cu" "B.Paste" "B.Mask") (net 2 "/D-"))
  (pad "26" smd rect (at 1.8 -3.45 45) (size 0.2 0.85) (layers "B.Cu" "B.Paste" "B.Mask") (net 3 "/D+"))
  (pad "27" smd rect (at 2.2 -3.45 45) (size 0.2 0.85) (layers "B.Cu" "B.Paste" "B.Mask") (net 9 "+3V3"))
  (pad "28" smd rect (at 2.6 -3.45 45) (size 0.2 0.85) (layers "B.Cu" "B.Paste" "B.Mask") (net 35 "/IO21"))
  (pad "29" smd rect (at 3.45 -2.6 315) (size 0.2 0.85) (layers "B.Cu" "B.Paste" "B.Mask") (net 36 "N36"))
  (pad "30" smd rect (at 3.45 -2.2 315) (size 0.2 0.85) (layers "B.Cu" "B.Paste" "B.Mask") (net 15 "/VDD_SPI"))
  (pad "31" smd rect (at 3.45 -1.8 315) (size 0.2 0.85) (layers "B.Cu" "B.Paste" "B.Mask") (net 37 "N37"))
  (pad "32" smd rect (at 3.45 -1.4 315) (size 0.2 0.85) (layers "B.Cu" "B.Paste" "B.Mask") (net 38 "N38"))
  (pad "33" smd rect (at 3.45 -1 315) (size 0.2 0.85) (layers "B.Cu" "B.Paste" "B.Mask") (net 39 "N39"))
  (pad "34" smd rect (at 3.45 -0.6 315) (size 0.2 0.85) (layers "B.Cu" "B.Paste" "B.Mask") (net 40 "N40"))
  (pad "35" smd rect (at 3.45 -0.2 315) (size 0.2 0.85) (layers "B.Cu" "B.Paste" "B.Mask") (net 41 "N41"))
  (pad "36" smd rect (at 3.45 0.2 315) (size 0.2 0.85) (layers "B.Cu" "B.Paste" "B.Mask") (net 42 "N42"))
  (pad "37" smd rect (at 3.45 0.6 315) (size 0.2 0.85) (layers "B.Cu" "B.Paste" "B.Mask") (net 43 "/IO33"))
  (pad "38" smd rect (at 3.45 1 315) (size 0.2 0.85) (layers "B.Cu" "B.Paste" "B.Mask") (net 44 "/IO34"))
  (pad "39" smd rect (at 3.45 1.4 315) (size 0.2 0.85) (layers "B.Cu" "B.Paste" "B.Mask") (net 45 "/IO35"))
  (pad "40" smd rect (at 3.45 1.8 315) (size 0.2 0.85) (layers "B.Cu" "B.Paste" "B.Mask") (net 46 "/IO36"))
  (pad "41" smd rect (at 3.45 2.2 315) (size 0.2 0.85) (layers "B.Cu" "B.Paste" "B.Mask") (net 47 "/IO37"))
  (pad "42" smd rect (at 3.45 2.6 315) (size 0.2 0.85) (layers "B.Cu" "B.Paste" "B.Mask") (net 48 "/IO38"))
  (pad "43" smd rect (at 2.6 3.45 45) (size 0.2 0.85) (layers "B.Cu" "B.Paste" "B.Mask") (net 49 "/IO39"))
  (pad "44" smd rect (at 2.2 3.45 45) (size 0.2 0.85) (layers "B.Cu" "B.Paste" "B.Mask") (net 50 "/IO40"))
  (pad "45" smd rect (at 1.8 3.45 45) (size 0.2 0.85) (layers "B.Cu" "B.Paste" "B.Mask") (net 9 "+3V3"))
  (pad "46" smd rect (at 1.4 3.45 45) (size 0.2 0.85) (layers "B.Cu" "B.Paste" "B.Mask") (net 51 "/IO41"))
  (pad "47" smd rect (at 1 3.45 45) (size 0.2 0.85) (layers "B.Cu" "B.Paste" "B.Mask") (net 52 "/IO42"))
  (pad "48" smd rect (at 0.6 3.45 45) (size 0.2 0.85) (layers "B.Cu" "B.Paste" "B.Mask") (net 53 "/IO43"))
  (pad "49" smd rect (at 0.2 3.45 45) (size 0.2 0.85) (layers "B.Cu" "B.Paste" "B.Mask") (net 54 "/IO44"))
  (pad "50" smd rect (at -0.2 3.45 45) (size 0.2 0.85) (layers "B.Cu" "B.Paste" "B.Mask") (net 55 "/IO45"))
  (pad "51" smd rect (at -0.6 3.45 45) (size 0.2 0.85) (layers "B.Cu" "B.Paste" "B.Mask") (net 9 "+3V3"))
  (pad "52" smd rect (at -1 3.45 45) (size 0.2 0.85) (layers "B.Cu" "B.Paste" "B.Mask") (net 13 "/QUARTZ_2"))
  (pad "53" smd rect (at -1.4 3.45 45) (size 0.2 0.85) (layers "B.Cu" "B.Paste" "B.Mask") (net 12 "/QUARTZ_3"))
  (pad "54" smd rect (at -1.8 3.45 45) (size 0.2 0.85) (layers "B.Cu" "B.Paste" "B.Mask") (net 9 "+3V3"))
  (pad "55" smd rect (at -2.2 3.45 45) (size 0.2 0.85) (layers "B.Cu" "B.Paste" "B.Mask") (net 6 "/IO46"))
  (pad "56" smd rect (at -2.6 3.45 45) (size 0.2 0.85) (layers "B.Cu" "B.Paste" "B.Mask") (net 5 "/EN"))
  (pad "57" smd rect (at 0 0 45) (size 4.05 4.05) (layers "B.Cu" "B.Paste" "B.Mask") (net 4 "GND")))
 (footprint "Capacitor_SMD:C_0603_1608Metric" (layer "B.Cu") (at 148.9 47.175 -90)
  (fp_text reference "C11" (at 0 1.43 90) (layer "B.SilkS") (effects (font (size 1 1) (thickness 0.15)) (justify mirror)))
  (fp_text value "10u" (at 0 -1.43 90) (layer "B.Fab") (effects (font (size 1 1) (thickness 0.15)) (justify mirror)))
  (pad "1" smd roundrect (at -0.775 0 270) (size 0.9 0.95) (layers "B.Cu" "B.Paste" "B.Mask") (roundrect_rratio 0.25) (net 9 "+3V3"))
  (pad "2" smd roundrect (at 0.775 0 270) (size 0.9 0.95) (layers "B.Cu" "B.Paste" "B.Mask") (roundrect_rratio 0.25) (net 4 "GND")))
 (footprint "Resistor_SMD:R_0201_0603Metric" (layer "B.Cu") (at 150.12 37)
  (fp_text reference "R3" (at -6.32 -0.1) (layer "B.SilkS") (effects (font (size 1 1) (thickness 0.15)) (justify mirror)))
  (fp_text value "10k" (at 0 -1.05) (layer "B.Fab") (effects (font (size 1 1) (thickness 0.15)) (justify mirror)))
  (pad "" smd roundrect (at -0.345 0) (size 0.318 0.36) (layers "B.Paste") (roundrect_rratio 0.25))
  (pad "" smd roundrect (at 0.345 0) (size 0.318 0.36) (layers "B.Paste") (roundrect_rratio 0.25))
  (pad "1" smd roundrect (at -0.32 0) (size 0.46 0.4) (layers "B.Cu" "B.Mask") (roundrect_rratio 0.25) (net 9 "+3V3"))
  (pad "2" smd roundrect (at 0.32 0) (size 0.46 0.4) (layers "B.Cu" "B.Mask") (roundrect_rratio 0.25) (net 34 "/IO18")))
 (gr_line (start 158.2 50.5) (end 158.2 33.2) (layer "Edge.Cuts") (width 0.1))
 (gr_line (start 158.2 33.2) (end 147.8 33.2) (layer "Edge.Cuts") (width 0.1))
 (gr_line (start 148.8 51.5) (end 157.2 51.5) (layer "Edge.Cuts") (width 0.1))
 (gr_line (start 147.8 33.2) (end 147.8 50.5) (layer "Edge.Cuts") (width 0.1))
 (gr_arc (start 148.8 51.5) (mid 148.092893 51.207107) (end 147.8 50.5) (layer "Edge.Cuts") (width 0.1))
 (gr_arc (start 158.2 50.5) (mid 157.907107 51.207107) (end 157.2 51.5) (layer "Edge.Cuts") (width 0.1))
 (segment (start 149.581472 38.68) (end 150.136218 39.234746) (width 0.09) (layer "B.Cu") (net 9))
 (segment (start 156.137171 44.337171) (end 155.238643 44.337171) (width 0.09) (layer "B.Cu") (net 9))
 (segment (start 156.760589 44.960589) (end 156.137171 44.337171) (width 0.09) (layer "B.Cu") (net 9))
 (segment (start 157.6 43.32) (end 157.6 43.304415) (width 0.09) (layer "B.Cu") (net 9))
 (segment (start 151.5 36.28) (end 151.5 36.63873) (width 0.09) (layer "B.Cu") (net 9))
 (segment (start 151.456174 45.339411) (end 150.439411 45.339411) (width 0.09) (layer "B.Cu") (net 9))
 (segment (start 148.9 45.678822) (end 149.239411 45.339411) (width 0.09) (layer "B.Cu") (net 9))
 (segment (start 148.5 38.68) (end 149.581472 38.68) (width 0.09) (layer "B.Cu") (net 9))
 (segment (start 157.6 43.304415) (end 156.712311 42.416726) (width 0.09) (layer "B.Cu") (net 9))
 (segment (start 152.6 46.8) (end 152.398959 46.598959) (width 0.09) (layer "B.Cu") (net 9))
 (segment (start 154.6 45.395585) (end 154.166726 44.962311) (width 0.09) (layer "B.Cu") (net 9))
 (segment (start 153.7 46.8) (end 154.6 45.9) (width 0.09) (layer "B.Cu") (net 9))
 (segment (start 152.398959 46.598959) (end 152.398959 45.527996) (width 0.09) (layer "B.Cu") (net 9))
 (segment (start 151.5 36.63873) (end 152.116117 37.254847) (width 0.09) (layer "B.Cu") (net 9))
 (segment (start 153.7 46.82) (end 153.7 46.8) (width 0.09) (layer "B.Cu") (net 9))
 (segment (start 155.238643 44.337171) (end 155.015254 44.113782) (width 0.09) (layer "B.Cu") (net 9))
 (segment (start 151.833274 44.962311) (end 151.456174 45.339411) (width 0.09) (layer "B.Cu") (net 9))
 (segment (start 154.6 45.9) (end 154.6 45.395585) (width 0.09) (layer "B.Cu") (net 9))
 (segment (start 150.890488 45.339411) (end 151.550431 44.679468) (width 0.09) (layer "B.Cu") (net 9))
 (segment (start 148.9 46.4) (end 148.9 45.678822) (width 0.09) (layer "B.Cu") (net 9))
 (segment (start 149.239411 45.339411) (end 150.890488 45.339411) (width 0.09) (layer "B.Cu") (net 9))
 (segment (start 150.5 37.335787) (end 151.267588 38.103375) (width 0.09) (layer "B.Cu") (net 34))
 (segment (start 150.5 37.02) (end 150.5 37.335787) (width 0.09) (layer "B.Cu") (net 34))
 (segment (start 154.178141 36.960589) (end 153.883883 37.254847) (width 0.09) (layer "B.Cu") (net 15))
 (segment (start 156.460589 36.960589) (end 154.178141 36.960589) (width 0.09) (layer "B.Cu") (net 15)))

